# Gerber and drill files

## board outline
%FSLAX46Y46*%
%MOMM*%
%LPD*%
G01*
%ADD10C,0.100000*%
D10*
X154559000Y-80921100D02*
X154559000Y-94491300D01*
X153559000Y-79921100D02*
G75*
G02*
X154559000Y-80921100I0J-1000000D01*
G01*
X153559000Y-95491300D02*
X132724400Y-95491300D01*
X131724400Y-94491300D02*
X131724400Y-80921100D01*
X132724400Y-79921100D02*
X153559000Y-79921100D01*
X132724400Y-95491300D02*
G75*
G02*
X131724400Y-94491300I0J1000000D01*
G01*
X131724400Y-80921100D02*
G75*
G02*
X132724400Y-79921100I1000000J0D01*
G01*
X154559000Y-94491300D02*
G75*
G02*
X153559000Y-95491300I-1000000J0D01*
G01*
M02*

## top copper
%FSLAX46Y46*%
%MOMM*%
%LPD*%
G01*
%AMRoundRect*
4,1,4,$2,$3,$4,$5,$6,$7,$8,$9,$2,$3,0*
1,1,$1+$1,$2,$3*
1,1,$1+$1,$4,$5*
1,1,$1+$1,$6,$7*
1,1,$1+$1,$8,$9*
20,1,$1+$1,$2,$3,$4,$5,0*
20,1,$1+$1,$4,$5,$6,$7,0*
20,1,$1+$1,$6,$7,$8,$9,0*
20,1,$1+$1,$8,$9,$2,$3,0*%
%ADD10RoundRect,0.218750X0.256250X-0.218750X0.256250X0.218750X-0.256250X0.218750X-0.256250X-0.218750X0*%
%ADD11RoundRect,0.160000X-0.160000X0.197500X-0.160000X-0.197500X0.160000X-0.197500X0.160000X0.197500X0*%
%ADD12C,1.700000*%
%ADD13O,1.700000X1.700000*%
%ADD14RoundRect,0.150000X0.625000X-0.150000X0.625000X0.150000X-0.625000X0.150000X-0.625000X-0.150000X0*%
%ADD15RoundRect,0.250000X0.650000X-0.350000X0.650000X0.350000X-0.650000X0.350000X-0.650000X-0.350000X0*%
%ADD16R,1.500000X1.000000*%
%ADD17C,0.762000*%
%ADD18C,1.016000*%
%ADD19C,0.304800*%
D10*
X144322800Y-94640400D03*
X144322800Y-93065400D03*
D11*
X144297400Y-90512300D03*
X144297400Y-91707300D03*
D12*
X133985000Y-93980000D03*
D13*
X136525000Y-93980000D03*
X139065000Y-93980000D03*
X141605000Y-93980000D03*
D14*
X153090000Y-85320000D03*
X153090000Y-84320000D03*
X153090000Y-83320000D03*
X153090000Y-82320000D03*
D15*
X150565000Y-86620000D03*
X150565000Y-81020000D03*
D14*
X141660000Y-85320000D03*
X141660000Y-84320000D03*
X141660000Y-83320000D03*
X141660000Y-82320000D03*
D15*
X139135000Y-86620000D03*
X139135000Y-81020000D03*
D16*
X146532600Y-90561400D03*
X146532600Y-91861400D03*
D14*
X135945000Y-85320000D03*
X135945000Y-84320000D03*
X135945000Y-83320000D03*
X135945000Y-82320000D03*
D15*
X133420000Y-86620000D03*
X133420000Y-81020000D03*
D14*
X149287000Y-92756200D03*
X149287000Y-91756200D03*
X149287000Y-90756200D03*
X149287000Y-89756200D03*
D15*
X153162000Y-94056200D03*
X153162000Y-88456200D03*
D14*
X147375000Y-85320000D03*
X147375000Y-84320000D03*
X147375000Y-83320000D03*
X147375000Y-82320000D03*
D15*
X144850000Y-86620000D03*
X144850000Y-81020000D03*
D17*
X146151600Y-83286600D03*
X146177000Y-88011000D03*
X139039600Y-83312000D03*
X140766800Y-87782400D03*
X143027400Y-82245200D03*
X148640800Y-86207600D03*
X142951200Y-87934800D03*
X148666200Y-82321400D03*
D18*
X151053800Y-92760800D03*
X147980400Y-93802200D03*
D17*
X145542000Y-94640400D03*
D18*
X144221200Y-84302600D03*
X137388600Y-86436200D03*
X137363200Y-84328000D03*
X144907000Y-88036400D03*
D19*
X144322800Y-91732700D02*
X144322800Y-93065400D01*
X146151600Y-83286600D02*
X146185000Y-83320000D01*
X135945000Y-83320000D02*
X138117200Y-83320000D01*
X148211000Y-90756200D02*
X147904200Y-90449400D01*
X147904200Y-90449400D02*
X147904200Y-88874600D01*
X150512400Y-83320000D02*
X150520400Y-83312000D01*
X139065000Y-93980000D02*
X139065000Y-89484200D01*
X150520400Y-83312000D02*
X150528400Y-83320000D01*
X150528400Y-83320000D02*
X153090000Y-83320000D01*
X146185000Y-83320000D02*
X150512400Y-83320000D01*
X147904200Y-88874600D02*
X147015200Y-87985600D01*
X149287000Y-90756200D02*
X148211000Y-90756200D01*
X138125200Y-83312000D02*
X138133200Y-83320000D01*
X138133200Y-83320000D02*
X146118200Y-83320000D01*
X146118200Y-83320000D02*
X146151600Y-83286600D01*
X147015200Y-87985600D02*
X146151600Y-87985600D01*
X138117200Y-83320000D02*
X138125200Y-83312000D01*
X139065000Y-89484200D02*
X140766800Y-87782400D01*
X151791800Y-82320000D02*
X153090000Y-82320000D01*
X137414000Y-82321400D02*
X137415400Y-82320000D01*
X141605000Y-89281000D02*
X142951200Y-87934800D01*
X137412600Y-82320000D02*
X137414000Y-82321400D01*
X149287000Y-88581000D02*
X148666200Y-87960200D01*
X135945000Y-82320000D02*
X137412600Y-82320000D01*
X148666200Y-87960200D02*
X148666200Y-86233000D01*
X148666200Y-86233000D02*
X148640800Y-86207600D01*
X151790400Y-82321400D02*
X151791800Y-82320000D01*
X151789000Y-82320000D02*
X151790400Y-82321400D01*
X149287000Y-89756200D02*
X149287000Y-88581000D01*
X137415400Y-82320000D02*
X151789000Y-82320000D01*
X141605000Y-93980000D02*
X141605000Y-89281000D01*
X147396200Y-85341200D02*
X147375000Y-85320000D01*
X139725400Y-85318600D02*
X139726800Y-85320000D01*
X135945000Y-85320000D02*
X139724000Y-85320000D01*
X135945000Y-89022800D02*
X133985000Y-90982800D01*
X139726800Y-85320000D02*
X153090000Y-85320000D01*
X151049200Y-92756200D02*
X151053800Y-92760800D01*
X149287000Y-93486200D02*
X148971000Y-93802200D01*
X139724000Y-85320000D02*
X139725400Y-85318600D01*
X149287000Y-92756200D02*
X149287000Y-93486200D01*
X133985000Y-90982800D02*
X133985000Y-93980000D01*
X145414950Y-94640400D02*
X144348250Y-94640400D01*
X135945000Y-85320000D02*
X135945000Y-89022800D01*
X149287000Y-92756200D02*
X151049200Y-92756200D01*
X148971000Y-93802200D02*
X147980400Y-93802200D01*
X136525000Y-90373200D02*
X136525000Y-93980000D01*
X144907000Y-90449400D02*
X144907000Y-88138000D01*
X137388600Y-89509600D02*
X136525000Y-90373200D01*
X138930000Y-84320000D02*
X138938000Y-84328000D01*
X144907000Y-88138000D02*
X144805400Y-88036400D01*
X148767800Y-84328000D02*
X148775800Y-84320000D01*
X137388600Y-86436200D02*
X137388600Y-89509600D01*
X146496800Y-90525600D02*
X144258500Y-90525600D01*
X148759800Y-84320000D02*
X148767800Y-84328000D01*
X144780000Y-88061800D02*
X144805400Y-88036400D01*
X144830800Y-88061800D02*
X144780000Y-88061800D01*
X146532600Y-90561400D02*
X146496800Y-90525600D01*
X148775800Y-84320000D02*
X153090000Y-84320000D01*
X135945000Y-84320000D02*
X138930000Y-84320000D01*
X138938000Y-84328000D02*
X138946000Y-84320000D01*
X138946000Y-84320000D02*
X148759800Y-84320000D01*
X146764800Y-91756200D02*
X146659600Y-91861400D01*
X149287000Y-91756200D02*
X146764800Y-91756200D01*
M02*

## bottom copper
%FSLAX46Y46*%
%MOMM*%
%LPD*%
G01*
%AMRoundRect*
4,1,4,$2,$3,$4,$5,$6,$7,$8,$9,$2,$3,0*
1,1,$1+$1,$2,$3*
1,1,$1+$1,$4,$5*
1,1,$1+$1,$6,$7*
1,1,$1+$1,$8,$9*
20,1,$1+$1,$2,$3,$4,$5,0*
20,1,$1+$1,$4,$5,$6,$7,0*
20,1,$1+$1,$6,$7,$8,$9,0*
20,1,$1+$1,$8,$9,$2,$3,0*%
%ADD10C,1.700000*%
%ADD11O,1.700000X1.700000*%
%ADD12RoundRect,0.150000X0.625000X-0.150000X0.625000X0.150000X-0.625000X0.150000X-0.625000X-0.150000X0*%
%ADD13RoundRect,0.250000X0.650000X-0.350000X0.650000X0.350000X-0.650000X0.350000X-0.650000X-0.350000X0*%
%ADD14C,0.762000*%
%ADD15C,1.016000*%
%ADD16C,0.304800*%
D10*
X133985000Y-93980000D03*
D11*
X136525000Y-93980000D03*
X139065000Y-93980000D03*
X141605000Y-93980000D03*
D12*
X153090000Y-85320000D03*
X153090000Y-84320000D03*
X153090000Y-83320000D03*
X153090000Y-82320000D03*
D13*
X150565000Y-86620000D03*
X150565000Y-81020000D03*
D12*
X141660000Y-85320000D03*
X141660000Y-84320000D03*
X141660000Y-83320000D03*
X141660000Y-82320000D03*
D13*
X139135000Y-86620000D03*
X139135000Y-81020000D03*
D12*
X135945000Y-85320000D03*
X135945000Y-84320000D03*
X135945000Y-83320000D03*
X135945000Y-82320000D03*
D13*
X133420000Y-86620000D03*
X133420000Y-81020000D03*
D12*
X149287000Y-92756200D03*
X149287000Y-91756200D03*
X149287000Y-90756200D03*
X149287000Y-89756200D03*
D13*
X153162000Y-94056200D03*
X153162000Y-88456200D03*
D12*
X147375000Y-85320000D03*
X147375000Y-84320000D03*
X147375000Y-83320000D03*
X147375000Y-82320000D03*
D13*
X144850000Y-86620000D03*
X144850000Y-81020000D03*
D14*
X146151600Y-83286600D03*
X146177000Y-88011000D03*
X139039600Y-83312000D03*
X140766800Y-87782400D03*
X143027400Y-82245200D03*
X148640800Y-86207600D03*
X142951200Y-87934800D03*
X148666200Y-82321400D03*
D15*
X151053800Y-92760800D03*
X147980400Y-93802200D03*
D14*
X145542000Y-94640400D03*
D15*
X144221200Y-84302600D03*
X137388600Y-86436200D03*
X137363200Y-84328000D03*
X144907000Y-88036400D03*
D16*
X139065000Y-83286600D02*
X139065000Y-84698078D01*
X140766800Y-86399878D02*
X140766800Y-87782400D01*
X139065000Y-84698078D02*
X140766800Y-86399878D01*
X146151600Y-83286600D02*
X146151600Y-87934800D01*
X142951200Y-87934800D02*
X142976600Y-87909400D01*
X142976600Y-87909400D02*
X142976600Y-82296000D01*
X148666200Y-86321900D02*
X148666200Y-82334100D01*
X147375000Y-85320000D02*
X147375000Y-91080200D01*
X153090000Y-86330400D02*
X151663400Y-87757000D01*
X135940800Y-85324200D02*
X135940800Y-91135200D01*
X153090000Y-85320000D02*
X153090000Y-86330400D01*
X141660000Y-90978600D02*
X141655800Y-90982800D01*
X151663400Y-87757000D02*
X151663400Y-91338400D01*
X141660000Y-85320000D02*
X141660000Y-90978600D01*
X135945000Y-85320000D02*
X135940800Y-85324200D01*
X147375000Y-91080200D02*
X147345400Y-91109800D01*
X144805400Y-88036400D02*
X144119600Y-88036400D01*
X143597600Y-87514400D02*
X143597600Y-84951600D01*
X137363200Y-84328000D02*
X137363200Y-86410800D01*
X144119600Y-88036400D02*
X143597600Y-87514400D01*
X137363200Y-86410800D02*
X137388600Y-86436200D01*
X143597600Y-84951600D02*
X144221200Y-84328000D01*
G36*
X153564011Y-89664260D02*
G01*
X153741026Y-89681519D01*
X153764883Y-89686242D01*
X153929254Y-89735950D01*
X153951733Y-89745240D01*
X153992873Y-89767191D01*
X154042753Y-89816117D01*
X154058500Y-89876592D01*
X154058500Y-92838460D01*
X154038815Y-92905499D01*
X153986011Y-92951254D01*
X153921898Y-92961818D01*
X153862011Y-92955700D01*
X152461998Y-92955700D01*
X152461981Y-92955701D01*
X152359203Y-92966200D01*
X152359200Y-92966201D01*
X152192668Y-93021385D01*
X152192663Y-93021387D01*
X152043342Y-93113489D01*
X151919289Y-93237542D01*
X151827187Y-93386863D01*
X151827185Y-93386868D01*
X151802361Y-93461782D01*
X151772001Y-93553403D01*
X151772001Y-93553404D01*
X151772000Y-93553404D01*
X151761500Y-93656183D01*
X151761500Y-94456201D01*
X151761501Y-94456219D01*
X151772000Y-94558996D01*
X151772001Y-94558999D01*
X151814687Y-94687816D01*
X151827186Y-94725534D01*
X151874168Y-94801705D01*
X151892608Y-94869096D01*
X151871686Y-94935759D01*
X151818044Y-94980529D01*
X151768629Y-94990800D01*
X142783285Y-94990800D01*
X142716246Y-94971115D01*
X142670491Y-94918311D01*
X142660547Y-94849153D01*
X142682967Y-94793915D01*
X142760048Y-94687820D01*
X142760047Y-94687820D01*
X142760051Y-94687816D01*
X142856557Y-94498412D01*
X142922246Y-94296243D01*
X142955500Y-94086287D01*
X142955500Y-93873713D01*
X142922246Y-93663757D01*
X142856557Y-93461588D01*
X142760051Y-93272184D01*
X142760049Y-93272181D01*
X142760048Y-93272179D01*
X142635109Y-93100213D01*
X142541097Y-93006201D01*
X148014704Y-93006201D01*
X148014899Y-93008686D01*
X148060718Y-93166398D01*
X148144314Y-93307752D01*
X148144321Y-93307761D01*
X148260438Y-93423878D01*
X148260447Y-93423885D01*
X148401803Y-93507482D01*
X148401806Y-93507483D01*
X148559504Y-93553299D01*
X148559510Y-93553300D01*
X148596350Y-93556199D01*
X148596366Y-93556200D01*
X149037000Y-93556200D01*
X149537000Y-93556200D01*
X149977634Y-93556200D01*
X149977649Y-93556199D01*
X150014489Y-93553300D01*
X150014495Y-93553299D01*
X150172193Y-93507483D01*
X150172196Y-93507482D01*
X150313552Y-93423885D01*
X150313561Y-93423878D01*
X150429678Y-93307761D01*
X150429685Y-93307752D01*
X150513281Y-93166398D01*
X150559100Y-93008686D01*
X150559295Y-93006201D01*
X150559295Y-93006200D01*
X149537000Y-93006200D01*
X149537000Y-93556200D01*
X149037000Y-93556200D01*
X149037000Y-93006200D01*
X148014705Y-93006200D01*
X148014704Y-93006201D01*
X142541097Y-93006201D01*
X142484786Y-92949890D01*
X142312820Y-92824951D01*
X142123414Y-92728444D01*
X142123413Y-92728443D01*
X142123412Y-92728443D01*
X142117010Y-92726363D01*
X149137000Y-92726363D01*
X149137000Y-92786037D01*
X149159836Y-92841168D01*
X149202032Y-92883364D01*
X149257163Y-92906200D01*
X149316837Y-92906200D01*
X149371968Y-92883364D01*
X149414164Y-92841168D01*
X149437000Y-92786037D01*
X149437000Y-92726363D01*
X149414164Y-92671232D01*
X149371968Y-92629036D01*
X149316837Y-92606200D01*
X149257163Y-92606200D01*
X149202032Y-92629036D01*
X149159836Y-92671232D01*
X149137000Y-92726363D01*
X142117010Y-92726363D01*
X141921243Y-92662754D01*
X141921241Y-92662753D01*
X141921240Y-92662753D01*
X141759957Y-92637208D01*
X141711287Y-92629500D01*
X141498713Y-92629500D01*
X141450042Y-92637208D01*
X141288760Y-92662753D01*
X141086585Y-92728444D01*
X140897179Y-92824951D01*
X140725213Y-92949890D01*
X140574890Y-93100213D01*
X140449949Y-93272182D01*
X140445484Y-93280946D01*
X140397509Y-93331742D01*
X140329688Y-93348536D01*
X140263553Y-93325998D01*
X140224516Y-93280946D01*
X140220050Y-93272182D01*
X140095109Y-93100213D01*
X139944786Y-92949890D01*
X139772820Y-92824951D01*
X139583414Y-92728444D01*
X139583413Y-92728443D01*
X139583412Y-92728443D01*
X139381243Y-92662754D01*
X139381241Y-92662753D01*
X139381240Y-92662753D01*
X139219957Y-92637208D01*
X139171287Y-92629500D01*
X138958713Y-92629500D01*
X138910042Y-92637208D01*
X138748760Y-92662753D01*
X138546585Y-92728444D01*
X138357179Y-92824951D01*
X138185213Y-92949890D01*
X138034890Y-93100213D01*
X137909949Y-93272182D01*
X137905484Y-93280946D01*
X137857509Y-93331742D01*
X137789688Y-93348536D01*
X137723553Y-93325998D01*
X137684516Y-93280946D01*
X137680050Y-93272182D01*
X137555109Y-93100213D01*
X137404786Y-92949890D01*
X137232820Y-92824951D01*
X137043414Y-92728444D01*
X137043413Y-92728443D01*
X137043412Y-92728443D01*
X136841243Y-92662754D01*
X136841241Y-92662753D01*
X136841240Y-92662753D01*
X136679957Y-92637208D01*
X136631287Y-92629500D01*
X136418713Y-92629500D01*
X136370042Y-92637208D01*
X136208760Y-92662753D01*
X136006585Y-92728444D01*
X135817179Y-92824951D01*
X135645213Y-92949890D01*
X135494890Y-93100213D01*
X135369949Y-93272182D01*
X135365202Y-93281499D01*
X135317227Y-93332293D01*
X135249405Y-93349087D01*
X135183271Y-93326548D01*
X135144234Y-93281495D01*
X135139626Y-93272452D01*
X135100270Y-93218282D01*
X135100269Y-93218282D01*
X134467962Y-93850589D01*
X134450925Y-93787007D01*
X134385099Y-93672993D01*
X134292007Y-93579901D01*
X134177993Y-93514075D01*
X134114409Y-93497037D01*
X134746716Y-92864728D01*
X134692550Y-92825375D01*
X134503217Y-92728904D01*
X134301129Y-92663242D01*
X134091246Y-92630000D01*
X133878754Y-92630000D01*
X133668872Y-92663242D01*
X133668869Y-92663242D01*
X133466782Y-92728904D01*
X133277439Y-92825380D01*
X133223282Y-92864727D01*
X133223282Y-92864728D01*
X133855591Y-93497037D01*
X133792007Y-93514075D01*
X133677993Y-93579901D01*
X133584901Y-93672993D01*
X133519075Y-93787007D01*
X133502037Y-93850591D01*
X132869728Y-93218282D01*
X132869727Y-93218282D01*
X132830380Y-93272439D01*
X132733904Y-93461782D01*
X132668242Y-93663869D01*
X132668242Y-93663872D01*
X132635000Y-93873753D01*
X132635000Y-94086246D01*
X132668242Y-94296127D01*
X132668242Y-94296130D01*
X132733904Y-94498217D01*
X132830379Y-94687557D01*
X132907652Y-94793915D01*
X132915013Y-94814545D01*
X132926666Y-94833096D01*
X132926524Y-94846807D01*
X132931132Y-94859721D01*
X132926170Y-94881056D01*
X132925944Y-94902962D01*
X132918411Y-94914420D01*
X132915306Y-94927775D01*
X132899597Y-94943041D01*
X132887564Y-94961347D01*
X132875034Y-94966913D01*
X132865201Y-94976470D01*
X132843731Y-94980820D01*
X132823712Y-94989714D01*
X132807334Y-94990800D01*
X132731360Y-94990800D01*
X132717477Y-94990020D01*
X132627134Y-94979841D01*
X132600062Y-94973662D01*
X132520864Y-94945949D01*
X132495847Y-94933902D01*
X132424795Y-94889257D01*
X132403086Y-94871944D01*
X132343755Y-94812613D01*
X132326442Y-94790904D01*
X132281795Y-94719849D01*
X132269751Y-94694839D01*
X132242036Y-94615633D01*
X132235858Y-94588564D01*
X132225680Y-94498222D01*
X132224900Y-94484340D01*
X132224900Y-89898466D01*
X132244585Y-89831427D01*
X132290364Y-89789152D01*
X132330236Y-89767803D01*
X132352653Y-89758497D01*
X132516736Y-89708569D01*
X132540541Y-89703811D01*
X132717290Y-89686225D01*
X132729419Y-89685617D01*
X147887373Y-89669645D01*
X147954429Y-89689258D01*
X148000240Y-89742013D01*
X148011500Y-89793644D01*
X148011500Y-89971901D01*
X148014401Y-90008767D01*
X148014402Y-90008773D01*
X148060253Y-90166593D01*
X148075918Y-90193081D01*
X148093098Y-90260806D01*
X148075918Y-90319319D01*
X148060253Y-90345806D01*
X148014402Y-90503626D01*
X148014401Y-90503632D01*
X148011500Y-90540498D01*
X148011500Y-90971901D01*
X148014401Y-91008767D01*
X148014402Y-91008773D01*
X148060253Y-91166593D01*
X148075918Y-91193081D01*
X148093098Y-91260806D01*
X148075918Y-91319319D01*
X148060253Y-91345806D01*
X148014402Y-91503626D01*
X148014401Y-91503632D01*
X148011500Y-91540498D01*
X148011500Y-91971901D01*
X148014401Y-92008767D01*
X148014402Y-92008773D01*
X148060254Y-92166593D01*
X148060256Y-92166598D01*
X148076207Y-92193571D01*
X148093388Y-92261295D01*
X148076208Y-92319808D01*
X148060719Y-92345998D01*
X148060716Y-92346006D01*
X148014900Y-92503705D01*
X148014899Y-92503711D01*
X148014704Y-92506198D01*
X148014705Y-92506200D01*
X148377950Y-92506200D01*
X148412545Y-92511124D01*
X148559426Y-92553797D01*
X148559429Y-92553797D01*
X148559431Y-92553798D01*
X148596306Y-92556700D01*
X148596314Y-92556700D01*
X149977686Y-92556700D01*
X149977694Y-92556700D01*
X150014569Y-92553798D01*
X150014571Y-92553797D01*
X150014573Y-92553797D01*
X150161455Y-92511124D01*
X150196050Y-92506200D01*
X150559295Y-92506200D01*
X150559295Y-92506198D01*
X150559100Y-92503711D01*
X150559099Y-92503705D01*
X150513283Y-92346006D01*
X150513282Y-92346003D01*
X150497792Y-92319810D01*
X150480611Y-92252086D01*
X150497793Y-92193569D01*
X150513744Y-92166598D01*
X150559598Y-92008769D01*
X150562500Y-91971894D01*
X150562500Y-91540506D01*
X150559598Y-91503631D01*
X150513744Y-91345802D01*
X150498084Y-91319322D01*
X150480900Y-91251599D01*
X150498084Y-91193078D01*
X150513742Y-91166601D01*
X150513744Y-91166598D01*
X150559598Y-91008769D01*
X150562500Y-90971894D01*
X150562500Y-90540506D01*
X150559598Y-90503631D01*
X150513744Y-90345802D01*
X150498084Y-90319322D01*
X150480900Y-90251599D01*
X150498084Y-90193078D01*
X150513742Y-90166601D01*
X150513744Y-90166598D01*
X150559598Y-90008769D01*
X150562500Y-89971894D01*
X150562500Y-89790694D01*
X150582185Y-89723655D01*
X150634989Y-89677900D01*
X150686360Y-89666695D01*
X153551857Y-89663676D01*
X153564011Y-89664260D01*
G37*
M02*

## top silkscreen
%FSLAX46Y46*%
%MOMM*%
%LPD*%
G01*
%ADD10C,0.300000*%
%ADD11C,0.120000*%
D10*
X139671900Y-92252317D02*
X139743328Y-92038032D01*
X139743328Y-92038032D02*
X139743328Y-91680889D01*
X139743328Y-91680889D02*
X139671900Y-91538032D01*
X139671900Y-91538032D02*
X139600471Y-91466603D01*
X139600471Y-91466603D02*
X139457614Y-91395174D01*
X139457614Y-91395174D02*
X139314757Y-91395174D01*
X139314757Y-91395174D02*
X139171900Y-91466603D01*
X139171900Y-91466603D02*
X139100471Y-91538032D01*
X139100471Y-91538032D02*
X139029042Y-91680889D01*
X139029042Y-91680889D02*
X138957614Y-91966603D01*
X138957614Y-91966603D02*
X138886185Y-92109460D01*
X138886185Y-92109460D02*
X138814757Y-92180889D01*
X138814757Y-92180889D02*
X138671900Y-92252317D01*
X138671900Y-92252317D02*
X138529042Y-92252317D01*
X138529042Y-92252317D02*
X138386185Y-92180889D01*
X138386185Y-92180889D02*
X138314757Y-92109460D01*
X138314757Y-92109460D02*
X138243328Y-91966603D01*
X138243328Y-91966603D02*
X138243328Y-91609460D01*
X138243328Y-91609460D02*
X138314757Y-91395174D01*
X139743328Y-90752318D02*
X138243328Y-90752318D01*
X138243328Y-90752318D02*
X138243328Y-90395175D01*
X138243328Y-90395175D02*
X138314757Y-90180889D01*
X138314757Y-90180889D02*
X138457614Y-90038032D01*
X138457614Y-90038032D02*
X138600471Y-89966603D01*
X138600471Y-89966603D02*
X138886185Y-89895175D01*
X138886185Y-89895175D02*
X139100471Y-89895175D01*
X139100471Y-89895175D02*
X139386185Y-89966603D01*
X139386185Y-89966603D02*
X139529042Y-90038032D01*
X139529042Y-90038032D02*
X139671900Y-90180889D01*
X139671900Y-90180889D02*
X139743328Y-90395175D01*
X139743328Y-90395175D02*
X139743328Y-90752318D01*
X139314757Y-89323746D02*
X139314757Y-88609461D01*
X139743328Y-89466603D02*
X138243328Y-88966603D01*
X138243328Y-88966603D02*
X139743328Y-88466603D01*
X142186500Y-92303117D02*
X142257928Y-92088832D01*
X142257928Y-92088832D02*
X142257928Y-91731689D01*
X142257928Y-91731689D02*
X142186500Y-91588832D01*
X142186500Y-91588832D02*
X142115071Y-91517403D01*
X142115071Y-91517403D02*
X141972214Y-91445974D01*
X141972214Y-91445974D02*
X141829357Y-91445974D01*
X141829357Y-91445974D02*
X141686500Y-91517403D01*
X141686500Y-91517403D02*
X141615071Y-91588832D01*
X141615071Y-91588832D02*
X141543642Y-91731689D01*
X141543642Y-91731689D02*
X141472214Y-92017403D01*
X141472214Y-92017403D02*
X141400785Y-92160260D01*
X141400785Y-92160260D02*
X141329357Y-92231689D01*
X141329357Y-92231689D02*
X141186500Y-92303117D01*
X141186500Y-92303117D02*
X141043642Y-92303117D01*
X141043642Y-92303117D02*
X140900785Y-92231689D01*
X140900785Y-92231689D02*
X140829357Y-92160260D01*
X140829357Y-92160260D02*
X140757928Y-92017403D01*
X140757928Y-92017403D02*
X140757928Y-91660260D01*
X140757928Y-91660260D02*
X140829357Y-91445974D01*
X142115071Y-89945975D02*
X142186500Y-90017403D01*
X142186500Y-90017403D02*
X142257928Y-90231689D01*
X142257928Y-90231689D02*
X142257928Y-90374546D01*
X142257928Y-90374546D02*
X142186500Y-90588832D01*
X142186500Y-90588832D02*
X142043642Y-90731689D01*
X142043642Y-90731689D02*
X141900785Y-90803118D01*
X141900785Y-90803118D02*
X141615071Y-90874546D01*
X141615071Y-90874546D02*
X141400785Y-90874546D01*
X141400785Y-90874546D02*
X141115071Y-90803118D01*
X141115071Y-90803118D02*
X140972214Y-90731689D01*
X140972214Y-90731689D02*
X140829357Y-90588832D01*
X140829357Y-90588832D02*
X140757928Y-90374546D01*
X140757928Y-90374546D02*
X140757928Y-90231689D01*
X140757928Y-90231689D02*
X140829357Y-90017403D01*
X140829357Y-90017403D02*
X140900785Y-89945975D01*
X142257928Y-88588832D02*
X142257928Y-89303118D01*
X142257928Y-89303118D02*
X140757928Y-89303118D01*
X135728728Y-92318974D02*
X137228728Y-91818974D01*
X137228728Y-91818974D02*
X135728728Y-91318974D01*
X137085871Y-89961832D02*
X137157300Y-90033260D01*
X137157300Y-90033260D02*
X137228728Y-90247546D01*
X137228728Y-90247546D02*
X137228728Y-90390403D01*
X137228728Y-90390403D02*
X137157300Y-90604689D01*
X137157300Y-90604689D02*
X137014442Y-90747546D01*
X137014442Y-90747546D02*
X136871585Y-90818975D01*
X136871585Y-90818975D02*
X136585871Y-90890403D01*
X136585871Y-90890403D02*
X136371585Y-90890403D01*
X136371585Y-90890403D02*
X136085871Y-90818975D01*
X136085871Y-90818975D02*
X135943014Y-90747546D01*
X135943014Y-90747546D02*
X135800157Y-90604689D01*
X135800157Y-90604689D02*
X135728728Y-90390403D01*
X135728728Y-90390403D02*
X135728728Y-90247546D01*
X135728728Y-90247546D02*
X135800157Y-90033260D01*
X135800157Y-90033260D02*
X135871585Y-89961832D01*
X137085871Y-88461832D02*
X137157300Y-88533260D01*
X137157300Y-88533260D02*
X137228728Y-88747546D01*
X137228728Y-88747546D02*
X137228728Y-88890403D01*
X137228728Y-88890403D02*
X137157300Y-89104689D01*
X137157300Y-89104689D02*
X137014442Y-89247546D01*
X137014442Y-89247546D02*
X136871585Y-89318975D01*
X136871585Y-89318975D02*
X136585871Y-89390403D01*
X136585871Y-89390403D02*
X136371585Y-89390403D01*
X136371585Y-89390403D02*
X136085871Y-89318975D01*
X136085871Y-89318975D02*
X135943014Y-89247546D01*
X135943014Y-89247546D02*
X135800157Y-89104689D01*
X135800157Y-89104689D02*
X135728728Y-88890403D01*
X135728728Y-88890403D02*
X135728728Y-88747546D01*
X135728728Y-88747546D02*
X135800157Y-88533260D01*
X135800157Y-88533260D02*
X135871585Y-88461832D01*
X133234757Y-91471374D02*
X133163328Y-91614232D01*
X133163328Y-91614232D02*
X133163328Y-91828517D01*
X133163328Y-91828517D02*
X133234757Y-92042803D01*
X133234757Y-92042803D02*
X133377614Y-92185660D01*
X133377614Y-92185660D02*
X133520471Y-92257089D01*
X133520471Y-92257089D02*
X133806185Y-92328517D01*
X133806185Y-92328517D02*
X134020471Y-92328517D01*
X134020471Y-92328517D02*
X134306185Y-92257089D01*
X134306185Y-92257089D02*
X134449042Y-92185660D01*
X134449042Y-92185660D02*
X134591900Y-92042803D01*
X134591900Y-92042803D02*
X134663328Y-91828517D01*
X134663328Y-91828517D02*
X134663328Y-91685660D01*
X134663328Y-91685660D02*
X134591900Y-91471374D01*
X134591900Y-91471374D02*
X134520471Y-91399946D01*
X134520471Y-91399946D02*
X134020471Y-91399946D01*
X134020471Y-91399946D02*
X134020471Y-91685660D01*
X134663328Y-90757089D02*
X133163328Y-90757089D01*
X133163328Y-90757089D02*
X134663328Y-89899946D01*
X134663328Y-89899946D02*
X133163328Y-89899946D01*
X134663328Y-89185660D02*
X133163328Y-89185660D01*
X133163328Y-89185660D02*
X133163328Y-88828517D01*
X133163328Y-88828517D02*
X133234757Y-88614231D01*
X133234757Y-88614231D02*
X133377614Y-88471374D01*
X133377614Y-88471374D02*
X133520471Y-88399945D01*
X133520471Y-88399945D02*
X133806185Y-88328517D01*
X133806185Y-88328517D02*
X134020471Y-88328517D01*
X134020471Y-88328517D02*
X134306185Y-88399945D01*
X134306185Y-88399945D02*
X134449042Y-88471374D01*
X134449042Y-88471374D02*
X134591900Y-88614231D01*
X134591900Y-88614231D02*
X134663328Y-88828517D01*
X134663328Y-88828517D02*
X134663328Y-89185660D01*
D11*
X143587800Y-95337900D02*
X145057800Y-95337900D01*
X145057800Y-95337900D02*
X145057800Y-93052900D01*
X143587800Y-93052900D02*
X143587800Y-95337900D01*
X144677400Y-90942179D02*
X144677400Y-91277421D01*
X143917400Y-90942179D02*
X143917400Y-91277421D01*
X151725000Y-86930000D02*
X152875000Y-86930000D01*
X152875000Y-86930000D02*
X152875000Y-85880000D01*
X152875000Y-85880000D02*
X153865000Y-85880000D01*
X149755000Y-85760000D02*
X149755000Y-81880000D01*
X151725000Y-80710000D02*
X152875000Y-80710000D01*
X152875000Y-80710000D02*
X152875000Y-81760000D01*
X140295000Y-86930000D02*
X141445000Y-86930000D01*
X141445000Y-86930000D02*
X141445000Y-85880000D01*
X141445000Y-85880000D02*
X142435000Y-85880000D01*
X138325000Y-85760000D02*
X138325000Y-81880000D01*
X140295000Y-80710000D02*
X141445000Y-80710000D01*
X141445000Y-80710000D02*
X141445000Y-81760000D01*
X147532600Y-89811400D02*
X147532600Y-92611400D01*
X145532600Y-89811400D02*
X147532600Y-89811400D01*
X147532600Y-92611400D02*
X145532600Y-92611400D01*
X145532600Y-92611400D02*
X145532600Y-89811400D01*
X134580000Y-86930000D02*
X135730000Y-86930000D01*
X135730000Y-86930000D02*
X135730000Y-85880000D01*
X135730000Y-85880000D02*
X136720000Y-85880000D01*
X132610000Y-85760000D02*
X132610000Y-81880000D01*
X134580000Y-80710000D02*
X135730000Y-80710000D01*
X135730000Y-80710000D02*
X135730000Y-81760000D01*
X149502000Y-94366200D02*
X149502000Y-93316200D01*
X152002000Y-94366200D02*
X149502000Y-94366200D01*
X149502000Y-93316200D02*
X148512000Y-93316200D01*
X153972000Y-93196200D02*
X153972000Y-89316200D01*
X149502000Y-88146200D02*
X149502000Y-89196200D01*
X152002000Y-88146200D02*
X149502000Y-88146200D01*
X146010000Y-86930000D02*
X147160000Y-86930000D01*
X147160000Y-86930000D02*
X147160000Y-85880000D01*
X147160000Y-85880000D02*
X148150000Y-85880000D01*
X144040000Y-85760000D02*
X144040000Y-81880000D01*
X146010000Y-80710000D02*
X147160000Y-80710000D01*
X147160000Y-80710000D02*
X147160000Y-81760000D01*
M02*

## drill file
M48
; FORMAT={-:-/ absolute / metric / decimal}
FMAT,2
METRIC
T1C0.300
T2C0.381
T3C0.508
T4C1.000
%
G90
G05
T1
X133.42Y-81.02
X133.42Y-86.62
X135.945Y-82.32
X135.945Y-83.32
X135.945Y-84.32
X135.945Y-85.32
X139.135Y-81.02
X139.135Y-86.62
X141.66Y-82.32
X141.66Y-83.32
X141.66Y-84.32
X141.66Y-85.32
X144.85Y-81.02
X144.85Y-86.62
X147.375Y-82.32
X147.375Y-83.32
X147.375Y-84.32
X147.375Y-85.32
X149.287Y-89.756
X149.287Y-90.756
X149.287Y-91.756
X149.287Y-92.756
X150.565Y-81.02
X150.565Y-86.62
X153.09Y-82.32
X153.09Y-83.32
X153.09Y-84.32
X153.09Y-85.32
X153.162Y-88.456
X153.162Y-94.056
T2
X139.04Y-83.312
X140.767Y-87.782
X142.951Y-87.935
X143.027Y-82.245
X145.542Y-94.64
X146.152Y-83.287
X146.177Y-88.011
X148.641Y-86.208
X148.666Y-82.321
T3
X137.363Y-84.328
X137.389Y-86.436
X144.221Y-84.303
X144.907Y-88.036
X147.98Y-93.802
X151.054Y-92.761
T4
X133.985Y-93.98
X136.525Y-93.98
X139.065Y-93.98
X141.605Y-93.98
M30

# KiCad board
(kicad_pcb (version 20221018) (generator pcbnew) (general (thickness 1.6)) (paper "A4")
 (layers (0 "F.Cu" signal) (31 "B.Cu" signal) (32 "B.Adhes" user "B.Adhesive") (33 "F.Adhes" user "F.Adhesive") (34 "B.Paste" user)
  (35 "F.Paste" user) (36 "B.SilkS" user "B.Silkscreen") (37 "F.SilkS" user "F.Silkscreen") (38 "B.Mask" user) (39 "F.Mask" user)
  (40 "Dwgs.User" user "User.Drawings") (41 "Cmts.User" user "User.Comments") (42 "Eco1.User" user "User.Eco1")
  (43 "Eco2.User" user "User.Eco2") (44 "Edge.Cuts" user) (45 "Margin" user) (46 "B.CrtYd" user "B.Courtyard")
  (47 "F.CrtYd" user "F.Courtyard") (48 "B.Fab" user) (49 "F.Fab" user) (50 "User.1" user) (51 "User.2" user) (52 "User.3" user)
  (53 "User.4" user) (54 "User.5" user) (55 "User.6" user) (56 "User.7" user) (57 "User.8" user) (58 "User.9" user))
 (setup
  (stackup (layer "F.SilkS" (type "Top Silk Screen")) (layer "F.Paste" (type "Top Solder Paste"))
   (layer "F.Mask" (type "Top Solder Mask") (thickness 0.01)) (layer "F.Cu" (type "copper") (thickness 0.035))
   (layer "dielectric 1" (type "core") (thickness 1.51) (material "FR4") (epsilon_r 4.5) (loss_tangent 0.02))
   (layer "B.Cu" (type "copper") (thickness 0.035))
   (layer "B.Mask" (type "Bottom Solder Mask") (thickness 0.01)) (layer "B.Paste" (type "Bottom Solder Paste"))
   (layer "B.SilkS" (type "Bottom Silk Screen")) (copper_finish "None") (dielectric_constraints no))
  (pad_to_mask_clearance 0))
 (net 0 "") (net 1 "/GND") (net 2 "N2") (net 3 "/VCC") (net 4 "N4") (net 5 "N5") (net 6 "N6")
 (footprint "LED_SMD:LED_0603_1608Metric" (layer "F.Cu") (at 144.3228 93.8529 90)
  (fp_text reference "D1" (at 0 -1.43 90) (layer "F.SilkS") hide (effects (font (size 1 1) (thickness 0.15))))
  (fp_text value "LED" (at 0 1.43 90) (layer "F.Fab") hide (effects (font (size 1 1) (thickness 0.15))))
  (fp_line (start -1.485 -0.735) (end -1.485 0.735) (stroke (width 0.12) (type solid)) (layer "F.SilkS"))
  (fp_line (start -1.485 0.735) (end 0.8 0.735) (stroke (width 0.12) (type solid)) (layer "F.SilkS"))
  (fp_line (start 0.8 -0.735) (end -1.485 -0.735) (stroke (width 0.12) (type solid)) (layer "F.SilkS"))
  (pad "1" smd roundrect (at -0.7875 0 90) (size 0.875 0.95) (layers "F.Cu" "F.Paste" "F.Mask") (roundrect_rratio 0.25) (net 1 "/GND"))
  (pad "2" smd roundrect (at 0.7875 0 90) (size 0.875 0.95) (layers "F.Cu" "F.Paste" "F.Mask") (roundrect_rratio 0.25) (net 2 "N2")))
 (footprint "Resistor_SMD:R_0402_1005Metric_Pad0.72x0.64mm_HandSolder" (layer "F.Cu") (at 144.2974 91.1098 -90)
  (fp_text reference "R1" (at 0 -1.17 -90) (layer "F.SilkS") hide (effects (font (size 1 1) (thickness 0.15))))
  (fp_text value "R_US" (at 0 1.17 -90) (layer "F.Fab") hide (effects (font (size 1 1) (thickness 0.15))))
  (fp_line (start -0.167621 -0.38) (end 0.167621 -0.38) (stroke (width 0.12) (type solid)) (layer "F.SilkS"))
  (fp_line (start -0.167621 0.38) (end 0.167621 0.38) (stroke (width 0.12) (type solid)) (layer "F.SilkS"))
  (pad "1" smd roundrect (at -0.5975 0 270) (size 0.715 0.64) (layers "F.Cu" "F.Paste" "F.Mask") (roundrect_rratio 0.25) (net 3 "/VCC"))
  (pad "2" smd roundrect (at 0.5975 0 270) (size 0.715 0.64) (layers "F.Cu" "F.Paste" "F.Mask") (roundrect_rratio 0.25) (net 2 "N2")))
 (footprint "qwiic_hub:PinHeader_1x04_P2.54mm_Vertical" (layer "F.Cu") (at 133.985 93.98 90)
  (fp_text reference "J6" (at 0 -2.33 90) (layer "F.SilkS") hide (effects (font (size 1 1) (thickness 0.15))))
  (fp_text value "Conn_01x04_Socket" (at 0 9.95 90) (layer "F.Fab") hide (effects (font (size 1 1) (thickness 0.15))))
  (pad "1" thru_hole circle (at 0 0 90) (size 1.7 1.7) (drill 1) (layers "*.Cu" "*.Mask") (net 1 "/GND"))
  (pad "2" thru_hole oval (at 0 2.54 90) (size 1.7 1.7) (drill 1) (layers "*.Cu" "*.Mask") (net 3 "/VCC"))
  (pad "3" thru_hole oval (at 0 5.08 90) (size 1.7 1.7) (drill 1) (layers "*.Cu" "*.Mask") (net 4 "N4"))
  (pad "4" thru_hole oval (at 0 7.62 90) (size 1.7 1.7) (drill 1) (layers "*.Cu" "*.Mask") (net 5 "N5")))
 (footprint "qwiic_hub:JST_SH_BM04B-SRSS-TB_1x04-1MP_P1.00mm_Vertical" (layer "F.Cu") (at 151.765 83.82 90)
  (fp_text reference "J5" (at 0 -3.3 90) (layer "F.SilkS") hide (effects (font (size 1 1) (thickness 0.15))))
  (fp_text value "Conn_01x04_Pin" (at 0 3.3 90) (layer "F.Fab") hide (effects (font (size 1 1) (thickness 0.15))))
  (fp_line (start -3.11 -0.04) (end -3.11 1.11) (stroke (width 0.12) (type solid)) (layer "F.SilkS"))
  (fp_line (start -3.11 1.11) (end -2.06 1.11) (stroke (width 0.12) (type solid)) (layer "F.SilkS"))
  (fp_line (start -2.06 1.11) (end -2.06 2.1) (stroke (width 0.12) (type solid)) (layer "F.SilkS"))
  (fp_line (start -1.94 -2.01) (end 1.94 -2.01) (stroke (width 0.12) (type solid)) (layer "F.SilkS"))
  (fp_line (start 3.11 -0.04) (end 3.11 1.11) (stroke (width 0.12) (type solid)) (layer "F.SilkS"))
  (fp_line (start 3.11 1.11) (end 2.06 1.11) (stroke (width 0.12) (type solid)) (layer "F.SilkS"))
  (pad "1" thru_hole roundrect (at -1.5 1.325 90) (size 0.6 1.55) (drill 0.3) (layers "*.Cu" "F.Paste" "F.Mask") (roundrect_rratio 0.25)
   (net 1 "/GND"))
  (pad "2" thru_hole roundrect (at -0.5 1.325 90) (size 0.6 1.55) (drill 0.3) (layers "*.Cu" "F.Paste" "F.Mask") (roundrect_rratio 0.25)
   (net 3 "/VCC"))
  (pad "3" thru_hole roundrect (at 0.5 1.325 90) (size 0.6 1.55) (drill 0.3) (layers "*.Cu" "F.Paste" "F.Mask") (roundrect_rratio 0.25)
   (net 4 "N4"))
  (pad "4" thru_hole roundrect (at 1.5 1.325 90) (size 0.6 1.55) (drill 0.3) (layers "*.Cu" "F.Paste" "F.Mask") (roundrect_rratio 0.25)
   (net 5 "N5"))
  (pad "MP" thru_hole roundrect (at -2.8 -1.2 90) (size 1.2 1.8) (drill 0.3) (layers "*.Cu" "F.Paste" "F.Mask")
   (roundrect_rratio 0.2083333333))
  (pad "MP" thru_hole roundrect (at 2.8 -1.2 90) (size 1.2 1.8) (drill 0.3) (layers "*.Cu" "F.Paste" "F.Mask")
   (roundrect_rratio 0.2083333333)))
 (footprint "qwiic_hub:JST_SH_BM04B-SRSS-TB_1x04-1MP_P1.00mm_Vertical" (layer "F.Cu") (at 140.335 83.82 90)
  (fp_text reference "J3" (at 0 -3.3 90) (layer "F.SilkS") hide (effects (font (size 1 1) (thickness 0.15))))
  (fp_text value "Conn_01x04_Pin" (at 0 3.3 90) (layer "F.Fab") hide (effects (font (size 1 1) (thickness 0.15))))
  (fp_line (start -3.11 -0.04) (end -3.11 1.11) (stroke (width 0.12) (type solid)) (layer "F.SilkS"))
  (fp_line (start -3.11 1.11) (end -2.06 1.11) (stroke (width 0.12) (type solid)) (layer "F.SilkS"))
  (fp_line (start -2.06 1.11) (end -2.06 2.1) (stroke (width 0.12) (type solid)) (layer "F.SilkS"))
  (fp_line (start -1.94 -2.01) (end 1.94 -2.01) (stroke (width 0.12) (type solid)) (layer "F.SilkS"))
  (fp_line (start 3.11 -0.04) (end 3.11 1.11) (stroke (width 0.12) (type solid)) (layer "F.SilkS"))
  (fp_line (start 3.11 1.11) (end 2.06 1.11) (stroke (width 0.12) (type solid)) (layer "F.SilkS"))
  (pad "1" thru_hole roundrect (at -1.5 1.325 90) (size 0.6 1.55) (drill 0.3) (layers "*.Cu" "F.Paste" "F.Mask") (roundrect_rratio 0.25)
   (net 1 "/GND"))
  (pad "2" thru_hole roundrect (at -0.5 1.325 90) (size 0.6 1.55) (drill 0.3) (layers "*.Cu" "F.Paste" "F.Mask") (roundrect_rratio 0.25)
   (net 3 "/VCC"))
  (pad "3" thru_hole roundrect (at 0.5 1.325 90) (size 0.6 1.55) (drill 0.3) (layers "*.Cu" "F.Paste" "F.Mask") (roundrect_rratio 0.25)
   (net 4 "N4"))
  (pad "4" thru_hole roundrect (at 1.5 1.325 90) (size 0.6 1.55) (drill 0.3) (layers "*.Cu" "F.Paste" "F.Mask") (roundrect_rratio 0.25)
   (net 5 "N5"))
  (pad "MP" thru_hole roundrect (at -2.8 -1.2 90) (size 1.2 1.8) (drill 0.3) (layers "*.Cu" "F.Paste" "F.Mask")
   (roundrect_rratio 0.2083333333))
  (pad "MP" thru_hole roundrect (at 2.8 -1.2 90) (size 1.2 1.8) (drill 0.3) (layers "*.Cu" "F.Paste" "F.Mask")
   (roundrect_rratio 0.2083333333)))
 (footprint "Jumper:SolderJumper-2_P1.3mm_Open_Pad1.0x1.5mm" (layer "F.Cu") (at 146.5326 91.2114 -90)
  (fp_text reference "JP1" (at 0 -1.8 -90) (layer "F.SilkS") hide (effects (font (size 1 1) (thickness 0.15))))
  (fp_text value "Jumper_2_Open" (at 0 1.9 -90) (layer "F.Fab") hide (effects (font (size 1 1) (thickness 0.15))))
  (fp_line (start -1.4 -1) (end 1.4 -1) (stroke (width 0.12) (type solid)) (layer "F.SilkS"))
  (fp_line (start -1.4 1) (end -1.4 -1) (stroke (width 0.12) (type solid)) (layer "F.SilkS"))
  (fp_line (start 1.4 -1) (end 1.4 1) (stroke (width 0.12) (type solid)) (layer "F.SilkS"))
  (fp_line (start 1.4 1) (end -1.4 1) (stroke (width 0.12) (type solid)) (layer "F.SilkS"))
  (pad "1" smd rect (at -0.65 0 270) (size 1 1.5) (layers "F.Cu" "F.Mask") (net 3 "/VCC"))
  (pad "2" smd rect (at 0.65 0 270) (size 1 1.5) (layers "F.Cu" "F.Mask") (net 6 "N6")))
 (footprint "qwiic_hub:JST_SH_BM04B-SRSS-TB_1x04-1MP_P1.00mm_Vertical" (layer "F.Cu") (at 134.62 83.82 90)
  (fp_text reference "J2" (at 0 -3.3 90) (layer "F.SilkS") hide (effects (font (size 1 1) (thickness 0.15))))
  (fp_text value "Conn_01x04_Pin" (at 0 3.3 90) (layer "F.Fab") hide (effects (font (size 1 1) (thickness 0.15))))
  (fp_line (start -3.11 -0.04) (end -3.11 1.11) (stroke (width 0.12) (type solid)) (layer "F.SilkS"))
  (fp_line (start -3.11 1.11) (end -2.06 1.11) (stroke (width 0.12) (type solid)) (layer "F.SilkS"))
  (fp_line (start -2.06 1.11) (end -2.06 2.1) (stroke (width 0.12) (type solid)) (layer "F.SilkS"))
  (fp_line (start -1.94 -2.01) (end 1.94 -2.01) (stroke (width 0.12) (type solid)) (layer "F.SilkS"))
  (fp_line (start 3.11 -0.04) (end 3.11 1.11) (stroke (width 0.12) (type solid)) (layer "F.SilkS"))
  (fp_line (start 3.11 1.11) (end 2.06 1.11) (stroke (width 0.12) (type solid)) (layer "F.SilkS"))
  (pad "1" thru_hole roundrect (at -1.5 1.325 90) (size 0.6 1.55) (drill 0.3) (layers "*.Cu" "F.Paste" "F.Mask") (roundrect_rratio 0.25)
   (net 1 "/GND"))
  (pad "2" thru_hole roundrect (at -0.5 1.325 90) (size 0.6 1.55) (drill 0.3) (layers "*.Cu" "F.Paste" "F.Mask") (roundrect_rratio 0.25)
   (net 3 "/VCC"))
  (pad "3" thru_hole roundrect (at 0.5 1.325 90) (size 0.6 1.55) (drill 0.3) (layers "*.Cu" "F.Paste" "F.Mask") (roundrect_rratio 0.25)
   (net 4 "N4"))
  (pad "4" thru_hole roundrect (at 1.5 1.325 90) (size 0.6 1.55) (drill 0.3) (layers "*.Cu" "F.Paste" "F.Mask") (roundrect_rratio 0.25)
   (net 5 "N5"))
  (pad "MP" thru_hole roundrect (at -2.8 -1.2 90) (size 1.2 1.8) (drill 0.3) (layers "*.Cu" "F.Paste" "F.Mask")
   (roundrect_rratio 0.2083333333))
  (pad "MP" thru_hole roundrect (at 2.8 -1.2 90) (size 1.2 1.8) (drill 0.3) (layers "*.Cu" "F.Paste" "F.Mask")
   (roundrect_rratio 0.2083333333)))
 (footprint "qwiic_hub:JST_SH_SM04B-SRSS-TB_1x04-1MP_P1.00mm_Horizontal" (layer "F.Cu") (at 151.287 91.2562 90)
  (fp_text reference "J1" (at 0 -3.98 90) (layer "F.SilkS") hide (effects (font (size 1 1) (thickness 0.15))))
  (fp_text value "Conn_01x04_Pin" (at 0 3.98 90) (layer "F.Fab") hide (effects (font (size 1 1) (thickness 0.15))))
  (fp_line (start -3.11 -1.785) (end -2.06 -1.785) (stroke (width 0.12) (type solid)) (layer "F.SilkS"))
  (fp_line (start -3.11 0.715) (end -3.11 -1.785) (stroke (width 0.12) (type solid)) (layer "F.SilkS"))
  (fp_line (start -2.06 -1.785) (end -2.06 -2.775) (stroke (width 0.12) (type solid)) (layer "F.SilkS"))
  (fp_line (start -1.94 2.685) (end 1.94 2.685) (stroke (width 0.12) (type solid)) (layer "F.SilkS"))
  (fp_line (start 3.11 -1.785) (end 2.06 -1.785) (stroke (width 0.12) (type solid)) (layer "F.SilkS"))
  (fp_line (start 3.11 0.715) (end 3.11 -1.785) (stroke (width 0.12) (type solid)) (layer "F.SilkS"))
  (pad "1" thru_hole roundrect (at -1.5 -2 90) (size 0.6 1.55) (drill 0.3) (layers "*.Cu" "F.Paste" "F.Mask") (roundrect_rratio 0.25)
   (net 1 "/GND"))
  (pad "2" thru_hole roundrect (at -0.5 -2 90) (size 0.6 1.55) (drill 0.3) (layers "*.Cu" "F.Paste" "F.Mask") (roundrect_rratio 0.25)
   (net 6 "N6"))
  (pad "3" thru_hole roundrect (at 0.5 -2 90) (size 0.6 1.55) (drill 0.3) (layers "*.Cu" "F.Paste" "F.Mask") (roundrect_rratio 0.25)
   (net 4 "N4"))
  (pad "4" thru_hole roundrect (at 1.5 -2 90) (size 0.6 1.55) (drill 0.3) (layers "*.Cu" "F.Paste" "F.Mask") (roundrect_rratio 0.25)
   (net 5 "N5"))
  (pad "MP" thru_hole roundrect (at -2.8 1.875 90) (size 1.2 1.8) (drill 0.3) (layers "*.Cu" "F.Paste" "F.Mask")
   (roundrect_rratio 0.2083333333))
  (pad "MP" thru_hole roundrect (at 2.8 1.875 90) (size 1.2 1.8) (drill 0.3) (layers "*.Cu" "F.Paste" "F.Mask")
   (roundrect_rratio 0.2083333333)))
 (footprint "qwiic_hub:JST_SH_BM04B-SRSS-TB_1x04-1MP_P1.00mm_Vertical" (layer "F.Cu") (at 146.05 83.82 90)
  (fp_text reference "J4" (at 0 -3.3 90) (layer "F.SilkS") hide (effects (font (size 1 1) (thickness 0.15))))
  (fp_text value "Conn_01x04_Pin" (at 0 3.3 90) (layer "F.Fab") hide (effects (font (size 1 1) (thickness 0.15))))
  (fp_line (start -3.11 -0.04) (end -3.11 1.11) (stroke (width 0.12) (type solid)) (layer "F.SilkS"))
  (fp_line (start -3.11 1.11) (end -2.06 1.11) (stroke (width 0.12) (type solid)) (layer "F.SilkS"))
  (fp_line (start -2.06 1.11) (end -2.06 2.1) (stroke (width 0.12) (type solid)) (layer "F.SilkS"))
  (fp_line (start -1.94 -2.01) (end 1.94 -2.01) (stroke (width 0.12) (type solid)) (layer "F.SilkS"))
  (fp_line (start 3.11 -0.04) (end 3.11 1.11) (stroke (width 0.12) (type solid)) (layer "F.SilkS"))
  (fp_line (start 3.11 1.11) (end 2.06 1.11) (stroke (width 0.12) (type solid)) (layer "F.SilkS"))
  (pad "1" thru_hole roundrect (at -1.5 1.325 90) (size 0.6 1.55) (drill 0.3) (layers "*.Cu" "F.Paste" "F.Mask") (roundrect_rratio 0.25)
   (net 1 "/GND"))
  (pad "2" thru_hole roundrect (at -0.5 1.325 90) (size 0.6 1.55) (drill 0.3) (layers "*.Cu" "F.Paste" "F.Mask") (roundrect_rratio 0.25)
   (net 3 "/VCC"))
  (pad "3" thru_hole roundrect (at 0.5 1.325 90) (size 0.6 1.55) (drill 0.3) (layers "*.Cu" "F.Paste" "F.Mask") (roundrect_rratio 0.25)
   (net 4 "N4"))
  (pad "4" thru_hole roundrect (at 1.5 1.325 90) (size 0.6 1.55) (drill 0.3) (layers "*.Cu" "F.Paste" "F.Mask") (roundrect_rratio 0.25)
   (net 5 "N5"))
  (pad "MP" thru_hole roundrect (at -2.8 -1.2 90) (size 1.2 1.8) (drill 0.3) (layers "*.Cu" "F.Paste" "F.Mask")
   (roundrect_rratio 0.2083333333))
  (pad "MP" thru_hole roundrect (at 2.8 -1.2 90) (size 1.2 1.8) (drill 0.3) (layers "*.Cu" "F.Paste" "F.Mask")
   (roundrect_rratio 0.2083333333)))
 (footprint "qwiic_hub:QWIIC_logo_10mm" (layer "B.Cu") (at 137.862099 89.790206 180)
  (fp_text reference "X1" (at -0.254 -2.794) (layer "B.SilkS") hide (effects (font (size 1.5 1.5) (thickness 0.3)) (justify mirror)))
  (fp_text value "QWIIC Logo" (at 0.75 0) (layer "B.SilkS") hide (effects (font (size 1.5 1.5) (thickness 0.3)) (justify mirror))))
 (gr_line (start 154.559 80.9211) (end 154.559 94.4913) (stroke (width 0.1) (type default)) (layer "Edge.Cuts"))
 (gr_arc (start 153.559 79.9211) (mid 154.266107 80.213993) (end 154.559 80.9211) (stroke (width 0.1) (type default)) (layer "Edge.Cuts"))
 (gr_line (start 153.559 95.4913) (end 132.7244 95.4913) (stroke (width 0.1) (type default)) (layer "Edge.Cuts"))
 (gr_line (start 131.7244 94.4913) (end 131.7244 80.9211) (stroke (width 0.1) (type default)) (layer "Edge.Cuts"))
 (gr_line (start 132.7244 79.9211) (end 153.559 79.9211) (stroke (width 0.1) (type default)) (layer "Edge.Cuts"))
 (gr_arc (start 132.7244 95.4913) (mid 132.017293 95.198407) (end 131.7244 94.4913) (stroke (width 0.1) (type default)) (layer "Edge.Cuts"))
 (gr_arc (start 131.7244 80.9211) (mid 132.017293 80.213993) (end 132.7244 79.9211) (stroke (width 0.1) (type default)) (layer "Edge.Cuts"))
 (gr_arc (start 154.559 94.4913) (mid 154.266107 95.198407) (end 153.559 95.4913) (stroke (width 0.1) (type default)) (layer "Edge.Cuts"))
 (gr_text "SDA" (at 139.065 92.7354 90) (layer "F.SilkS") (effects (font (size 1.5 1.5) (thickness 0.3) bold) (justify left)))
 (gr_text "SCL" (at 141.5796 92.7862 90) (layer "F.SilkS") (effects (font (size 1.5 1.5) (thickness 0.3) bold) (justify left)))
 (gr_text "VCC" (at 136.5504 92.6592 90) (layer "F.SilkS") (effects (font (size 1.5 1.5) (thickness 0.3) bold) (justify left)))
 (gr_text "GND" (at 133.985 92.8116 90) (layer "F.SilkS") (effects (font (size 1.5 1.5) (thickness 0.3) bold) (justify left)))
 (segment (start 144.3228 91.7327) (end 144.3228 93.0654) (width 0.3048) (layer "F.Cu") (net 2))
 (segment (start 146.1516 83.2866) (end 146.185 83.32) (width 0.3048) (layer "F.Cu") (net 4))
 (segment (start 135.945 83.32) (end 138.1172 83.32) (width 0.3048) (layer "F.Cu") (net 4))
 (segment (start 148.211 90.7562) (end 147.9042 90.4494) (width 0.3048) (layer "F.Cu") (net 4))
 (segment (start 147.9042 90.4494) (end 147.9042 88.8746) (width 0.3048) (layer "F.Cu") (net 4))
 (segment (start 150.5124 83.32) (end 150.5204 83.312) (width 0.3048) (layer "F.Cu") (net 4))
 (segment (start 139.065 93.98) (end 139.065 89.4842) (width 0.3048) (layer "F.Cu") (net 4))
 (segment (start 150.5204 83.312) (end 150.5284 83.32) (width 0.3048) (layer "F.Cu") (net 4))
 (segment (start 150.5284 83.32) (end 153.09 83.32) (width 0.3048) (layer "F.Cu") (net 4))
 (segment (start 146.185 83.32) (end 150.5124 83.32) (width 0.3048) (layer "F.Cu") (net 4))
 (segment (start 147.9042 88.8746) (end 147.0152 87.9856) (width 0.3048) (layer "F.Cu") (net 4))
 (segment (start 149.287 90.7562) (end 148.211 90.7562) (width 0.3048) (layer "F.Cu") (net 4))
 (segment (start 138.1252 83.312) (end 138.1332 83.32) (width 0.3048) (layer "F.Cu") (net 4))
 (segment (start 138.1332 83.32) (end 146.1182 83.32) (width 0.3048) (layer "F.Cu") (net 4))
 (segment (start 146.1182 83.32) (end 146.1516 83.2866) (width 0.3048) (layer "F.Cu") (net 4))
 (segment (start 147.0152 87.9856) (end 146.1516 87.9856) (width 0.3048) (layer "F.Cu") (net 4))
 (segment (start 138.1172 83.32) (end 138.1252 83.312) (width 0.3048) (layer "F.Cu") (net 4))
 (segment (start 139.065 89.4842) (end 140.7668 87.7824) (width 0.3048) (layer "F.Cu") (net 4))
 (via (at 146.1516 83.2866) (size 0.762) (drill 0.381) (layers "F.Cu" "B.Cu") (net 4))
 (via (at 146.177 88.011) (size 0.762) (drill 0.381) (layers "F.Cu" "B.Cu") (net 4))
 (via (at 139.0396 83.312) (size 0.762) (drill 0.381) (layers "F.Cu" "B.Cu") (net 4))
 (via (at 140.7668 87.7824) (size 0.762) (drill 0.381) (layers "F.Cu" "B.Cu") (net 4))
 (segment (start 139.065 83.2866) (end 139.065 84.698078) (width 0.3048) (layer "B.Cu") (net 4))
 (segment (start 140.7668 86.399878) (end 140.7668 87.7824) (width 0.3048) (layer "B.Cu") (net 4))
 (segment (start 139.065 84.698078) (end 140.7668 86.399878) (width 0.3048) (layer "B.Cu") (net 4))
 (segment (start 146.1516 83.2866) (end 146.1516 87.9348) (width 0.3048) (layer "B.Cu") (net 4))
 (segment (start 151.7918 82.32) (end 153.09 82.32) (width 0.3048) (layer "F.Cu") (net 5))
 (segment (start 137.414 82.3214) (end 137.4154 82.32) (width 0.3048) (layer "F.Cu") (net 5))
 (segment (start 141.605 89.281) (end 142.9512 87.9348) (width 0.3048) (layer "F.Cu") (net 5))
 (segment (start 137.4126 82.32) (end 137.414 82.3214) (width 0.3048) (layer "F.Cu") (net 5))
 (segment (start 149.287 88.581) (end 148.6662 87.9602) (width 0.3048) (layer "F.Cu") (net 5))
 (segment (start 135.945 82.32) (end 137.4126 82.32) (width 0.3048) (layer "F.Cu") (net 5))
 (segment (start 148.6662 87.9602) (end 148.6662 86.233) (width 0.3048) (layer "F.Cu") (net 5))
 (segment (start 148.6662 86.233) (end 148.6408 86.2076) (width 0.3048) (layer "F.Cu") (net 5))
 (segment (start 151.7904 82.3214) (end 151.7918 82.32) (width 0.3048) (layer "F.Cu") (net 5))
 (segment (start 151.789 82.32) (end 151.7904 82.3214) (width 0.3048) (layer "F.Cu") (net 5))
 (segment (start 149.287 89.7562) (end 149.287 88.581) (width 0.3048) (layer "F.Cu") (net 5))
 (segment (start 137.4154 82.32) (end 151.789 82.32) (width 0.3048) (layer "F.Cu") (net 5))
 (segment (start 141.605 93.98) (end 141.605 89.281) (width 0.3048) (layer "F.Cu") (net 5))
 (via (at 143.0274 82.2452) (size 0.762) (drill 0.381) (layers "F.Cu" "B.Cu") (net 5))
 (via (at 148.6408 86.2076) (size 0.762) (drill 0.381) (layers "F.Cu" "B.Cu") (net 5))
 (via (at 142.9512 87.9348) (size 0.762) (drill 0.381) (layers "F.Cu" "B.Cu") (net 5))
 (via (at 148.6662 82.3214) (size 0.762) (drill 0.381) (layers "F.Cu" "B.Cu") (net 5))
 (segment (start 142.9512 87.9348) (end 142.9766 87.9094) (width 0.3048) (layer "B.Cu") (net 5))
 (segment (start 142.9766 87.9094) (end 142.9766 82.296) (width 0.3048) (layer "B.Cu") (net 5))
 (segment (start 148.6662 86.3219) (end 148.6662 82.3341) (width 0.3048) (layer "B.Cu") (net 5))
 (segment (start 147.3962 85.3412) (end 147.375 85.32) (width 0.3048) (layer "F.Cu") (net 1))
 (segment (start 139.7254 85.3186) (end 139.7268 85.32) (width 0.3048) (layer "F.Cu") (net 1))
 (segment (start 135.945 85.32) (end 139.724 85.32) (width 0.3048) (layer "F.Cu") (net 1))
 (segment (start 135.945 89.0228) (end 133.985 90.9828) (width 0.3048) (layer "F.Cu") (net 1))
 (segment (start 139.7268 85.32) (end 153.09 85.32) (width 0.3048) (layer "F.Cu") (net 1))
 (segment (start 151.0492 92.7562) (end 151.0538 92.7608) (width 0.3048) (layer "F.Cu") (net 1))
 (segment (start 149.287 93.4862) (end 148.971 93.8022) (width 0.3048) (layer "F.Cu") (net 1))
 (segment (start 139.724 85.32) (end 139.7254 85.3186) (width 0.3048) (layer "F.Cu") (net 1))
 (segment (start 149.287 92.7562) (end 149.287 93.4862) (width 0.3048) (layer "F.Cu") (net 1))
 (segment (start 133.985 90.9828) (end 133.985 93.98) (width 0.3048) (layer "F.Cu") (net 1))
 (segment (start 145.41495 94.6404) (end 144.34825 94.6404) (width 0.3048) (layer "F.Cu") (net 1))
 (segment (start 135.945 85.32) (end 135.945 89.0228) (width 0.3048) (layer "F.Cu") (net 1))
 (segment (start 149.287 92.7562) (end 151.0492 92.7562) (width 0.3048) (layer "F.Cu") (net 1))
 (segment (start 148.971 93.8022) (end 147.9804 93.8022) (width 0.3048) (layer "F.Cu") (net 1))
 (via (at 151.0538 92.7608) (size 1.016) (drill 0.508) (layers "F.Cu" "B.Cu") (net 1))
 (via (at 147.9804 93.8022) (size 1.016) (drill 0.508) (layers "F.Cu" "B.Cu") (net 1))
 (via (at 145.542 94.6404) (size 0.762) (drill 0.381) (layers "F.Cu" "B.Cu") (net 1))
 (segment (start 147.375 85.32) (end 147.375 91.0802) (width 0.3048) (layer "B.Cu") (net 1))
 (segment (start 153.09 86.3304) (end 151.6634 87.757) (width 0.3048) (layer "B.Cu") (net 1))
 (segment (start 135.9408 85.3242) (end 135.9408 91.1352) (width 0.3048) (layer "B.Cu") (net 1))
 (segment (start 153.09 85.32) (end 153.09 86.3304) (width 0.3048) (layer "B.Cu") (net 1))
 (segment (start 141.66 90.9786) (end 141.6558 90.9828) (width 0.3048) (layer "B.Cu") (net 1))
 (segment (start 151.6634 87.757) (end 151.6634 91.3384) (width 0.3048) (layer "B.Cu") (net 1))
 (segment (start 141.66 85.32) (end 141.66 90.9786) (width 0.3048) (layer "B.Cu") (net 1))
 (segment (start 135.945 85.32) (end 135.9408 85.3242) (width 0.3048) (layer "B.Cu") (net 1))
 (segment (start 147.375 91.0802) (end 147.3454 91.1098) (width 0.3048) (layer "B.Cu") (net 1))
 (segment (start 136.525 90.3732) (end 136.525 93.98) (width 0.3048) (layer "F.Cu") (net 3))
 (segment (start 144.907 90.4494) (end 144.907 88.138) (width 0.3048) (layer "F.Cu") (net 3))
 (segment (start 137.3886 89.5096) (end 136.525 90.3732) (width 0.3048) (layer "F.Cu") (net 3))
 (segment (start 138.93 84.32) (end 138.938 84.328) (width 0.3048) (layer "F.Cu") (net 3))
 (segment (start 144.907 88.138) (end 144.8054 88.0364) (width 0.3048) (layer "F.Cu") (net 3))
 (segment (start 148.7678 84.328) (end 148.7758 84.32) (width 0.3048) (layer "F.Cu") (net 3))
 (segment (start 137.3886 86.4362) (end 137.3886 89.5096) (width 0.3048) (layer "F.Cu") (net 3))
 (segment (start 146.4968 90.5256) (end 144.2585 90.5256) (width 0.3048) (layer "F.Cu") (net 3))
 (segment (start 148.7598 84.32) (end 148.7678 84.328) (width 0.3048) (layer "F.Cu") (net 3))
 (segment (start 144.78 88.0618) (end 144.8054 88.0364) (width 0.3048) (layer "F.Cu") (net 3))
 (segment (start 144.8308 88.0618) (end 144.78 88.0618) (width 0.3048) (layer "F.Cu") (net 3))
 (segment (start 146.5326 90.5614) (end 146.4968 90.5256) (width 0.3048) (layer "F.Cu") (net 3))
 (segment (start 148.7758 84.32) (end 153.09 84.32) (width 0.3048) (layer "F.Cu") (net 3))
 (segment (start 135.945 84.32) (end 138.93 84.32) (width 0.3048) (layer "F.Cu") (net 3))
 (segment (start 138.938 84.328) (end 138.946 84.32) (width 0.3048) (layer "F.Cu") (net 3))
 (segment (start 138.946 84.32) (end 148.7598 84.32) (width 0.3048) (layer "F.Cu") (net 3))
 (via (at 144.2212 84.3026) (size 1.016) (drill 0.508) (layers "F.Cu" "B.Cu") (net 3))
 (via (at 137.3886 86.4362) (size 1.016) (drill 0.508) (layers "F.Cu" "B.Cu") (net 3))
 (via (at 137.3632 84.328) (size 1.016) (drill 0.508) (layers "F.Cu" "B.Cu") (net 3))
 (via (at 144.907 88.0364) (size 1.016) (drill 0.508) (layers "F.Cu" "B.Cu") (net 3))
 (segment (start 144.8054 88.0364) (end 144.1196 88.0364) (width 0.3048) (layer "B.Cu") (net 3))
 (segment (start 143.5976 87.5144) (end 143.5976 84.9516) (width 0.3048) (layer "B.Cu") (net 3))
 (segment (start 137.3632 84.328) (end 137.3632 86.4108) (width 0.3048) (layer "B.Cu") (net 3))
 (segment (start 144.1196 88.0364) (end 143.5976 87.5144) (width 0.3048) (layer "B.Cu") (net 3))
 (segment (start 137.3632 86.4108) (end 137.3886 86.4362) (width 0.3048) (layer "B.Cu") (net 3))
 (segment (start 143.5976 84.9516) (end 144.2212 84.328) (width 0.3048) (layer "B.Cu") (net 3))
 (segment (start 146.7648 91.7562) (end 146.6596 91.8614) (width 0.3048) (layer "F.Cu") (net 6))
 (segment (start 149.287 91.7562) (end 146.7648 91.7562) (width 0.3048) (layer "F.Cu") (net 6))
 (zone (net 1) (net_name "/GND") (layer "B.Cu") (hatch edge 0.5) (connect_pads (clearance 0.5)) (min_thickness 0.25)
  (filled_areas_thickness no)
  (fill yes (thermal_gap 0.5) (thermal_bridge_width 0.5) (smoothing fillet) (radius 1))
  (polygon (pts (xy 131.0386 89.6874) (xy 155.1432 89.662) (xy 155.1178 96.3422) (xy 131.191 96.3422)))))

